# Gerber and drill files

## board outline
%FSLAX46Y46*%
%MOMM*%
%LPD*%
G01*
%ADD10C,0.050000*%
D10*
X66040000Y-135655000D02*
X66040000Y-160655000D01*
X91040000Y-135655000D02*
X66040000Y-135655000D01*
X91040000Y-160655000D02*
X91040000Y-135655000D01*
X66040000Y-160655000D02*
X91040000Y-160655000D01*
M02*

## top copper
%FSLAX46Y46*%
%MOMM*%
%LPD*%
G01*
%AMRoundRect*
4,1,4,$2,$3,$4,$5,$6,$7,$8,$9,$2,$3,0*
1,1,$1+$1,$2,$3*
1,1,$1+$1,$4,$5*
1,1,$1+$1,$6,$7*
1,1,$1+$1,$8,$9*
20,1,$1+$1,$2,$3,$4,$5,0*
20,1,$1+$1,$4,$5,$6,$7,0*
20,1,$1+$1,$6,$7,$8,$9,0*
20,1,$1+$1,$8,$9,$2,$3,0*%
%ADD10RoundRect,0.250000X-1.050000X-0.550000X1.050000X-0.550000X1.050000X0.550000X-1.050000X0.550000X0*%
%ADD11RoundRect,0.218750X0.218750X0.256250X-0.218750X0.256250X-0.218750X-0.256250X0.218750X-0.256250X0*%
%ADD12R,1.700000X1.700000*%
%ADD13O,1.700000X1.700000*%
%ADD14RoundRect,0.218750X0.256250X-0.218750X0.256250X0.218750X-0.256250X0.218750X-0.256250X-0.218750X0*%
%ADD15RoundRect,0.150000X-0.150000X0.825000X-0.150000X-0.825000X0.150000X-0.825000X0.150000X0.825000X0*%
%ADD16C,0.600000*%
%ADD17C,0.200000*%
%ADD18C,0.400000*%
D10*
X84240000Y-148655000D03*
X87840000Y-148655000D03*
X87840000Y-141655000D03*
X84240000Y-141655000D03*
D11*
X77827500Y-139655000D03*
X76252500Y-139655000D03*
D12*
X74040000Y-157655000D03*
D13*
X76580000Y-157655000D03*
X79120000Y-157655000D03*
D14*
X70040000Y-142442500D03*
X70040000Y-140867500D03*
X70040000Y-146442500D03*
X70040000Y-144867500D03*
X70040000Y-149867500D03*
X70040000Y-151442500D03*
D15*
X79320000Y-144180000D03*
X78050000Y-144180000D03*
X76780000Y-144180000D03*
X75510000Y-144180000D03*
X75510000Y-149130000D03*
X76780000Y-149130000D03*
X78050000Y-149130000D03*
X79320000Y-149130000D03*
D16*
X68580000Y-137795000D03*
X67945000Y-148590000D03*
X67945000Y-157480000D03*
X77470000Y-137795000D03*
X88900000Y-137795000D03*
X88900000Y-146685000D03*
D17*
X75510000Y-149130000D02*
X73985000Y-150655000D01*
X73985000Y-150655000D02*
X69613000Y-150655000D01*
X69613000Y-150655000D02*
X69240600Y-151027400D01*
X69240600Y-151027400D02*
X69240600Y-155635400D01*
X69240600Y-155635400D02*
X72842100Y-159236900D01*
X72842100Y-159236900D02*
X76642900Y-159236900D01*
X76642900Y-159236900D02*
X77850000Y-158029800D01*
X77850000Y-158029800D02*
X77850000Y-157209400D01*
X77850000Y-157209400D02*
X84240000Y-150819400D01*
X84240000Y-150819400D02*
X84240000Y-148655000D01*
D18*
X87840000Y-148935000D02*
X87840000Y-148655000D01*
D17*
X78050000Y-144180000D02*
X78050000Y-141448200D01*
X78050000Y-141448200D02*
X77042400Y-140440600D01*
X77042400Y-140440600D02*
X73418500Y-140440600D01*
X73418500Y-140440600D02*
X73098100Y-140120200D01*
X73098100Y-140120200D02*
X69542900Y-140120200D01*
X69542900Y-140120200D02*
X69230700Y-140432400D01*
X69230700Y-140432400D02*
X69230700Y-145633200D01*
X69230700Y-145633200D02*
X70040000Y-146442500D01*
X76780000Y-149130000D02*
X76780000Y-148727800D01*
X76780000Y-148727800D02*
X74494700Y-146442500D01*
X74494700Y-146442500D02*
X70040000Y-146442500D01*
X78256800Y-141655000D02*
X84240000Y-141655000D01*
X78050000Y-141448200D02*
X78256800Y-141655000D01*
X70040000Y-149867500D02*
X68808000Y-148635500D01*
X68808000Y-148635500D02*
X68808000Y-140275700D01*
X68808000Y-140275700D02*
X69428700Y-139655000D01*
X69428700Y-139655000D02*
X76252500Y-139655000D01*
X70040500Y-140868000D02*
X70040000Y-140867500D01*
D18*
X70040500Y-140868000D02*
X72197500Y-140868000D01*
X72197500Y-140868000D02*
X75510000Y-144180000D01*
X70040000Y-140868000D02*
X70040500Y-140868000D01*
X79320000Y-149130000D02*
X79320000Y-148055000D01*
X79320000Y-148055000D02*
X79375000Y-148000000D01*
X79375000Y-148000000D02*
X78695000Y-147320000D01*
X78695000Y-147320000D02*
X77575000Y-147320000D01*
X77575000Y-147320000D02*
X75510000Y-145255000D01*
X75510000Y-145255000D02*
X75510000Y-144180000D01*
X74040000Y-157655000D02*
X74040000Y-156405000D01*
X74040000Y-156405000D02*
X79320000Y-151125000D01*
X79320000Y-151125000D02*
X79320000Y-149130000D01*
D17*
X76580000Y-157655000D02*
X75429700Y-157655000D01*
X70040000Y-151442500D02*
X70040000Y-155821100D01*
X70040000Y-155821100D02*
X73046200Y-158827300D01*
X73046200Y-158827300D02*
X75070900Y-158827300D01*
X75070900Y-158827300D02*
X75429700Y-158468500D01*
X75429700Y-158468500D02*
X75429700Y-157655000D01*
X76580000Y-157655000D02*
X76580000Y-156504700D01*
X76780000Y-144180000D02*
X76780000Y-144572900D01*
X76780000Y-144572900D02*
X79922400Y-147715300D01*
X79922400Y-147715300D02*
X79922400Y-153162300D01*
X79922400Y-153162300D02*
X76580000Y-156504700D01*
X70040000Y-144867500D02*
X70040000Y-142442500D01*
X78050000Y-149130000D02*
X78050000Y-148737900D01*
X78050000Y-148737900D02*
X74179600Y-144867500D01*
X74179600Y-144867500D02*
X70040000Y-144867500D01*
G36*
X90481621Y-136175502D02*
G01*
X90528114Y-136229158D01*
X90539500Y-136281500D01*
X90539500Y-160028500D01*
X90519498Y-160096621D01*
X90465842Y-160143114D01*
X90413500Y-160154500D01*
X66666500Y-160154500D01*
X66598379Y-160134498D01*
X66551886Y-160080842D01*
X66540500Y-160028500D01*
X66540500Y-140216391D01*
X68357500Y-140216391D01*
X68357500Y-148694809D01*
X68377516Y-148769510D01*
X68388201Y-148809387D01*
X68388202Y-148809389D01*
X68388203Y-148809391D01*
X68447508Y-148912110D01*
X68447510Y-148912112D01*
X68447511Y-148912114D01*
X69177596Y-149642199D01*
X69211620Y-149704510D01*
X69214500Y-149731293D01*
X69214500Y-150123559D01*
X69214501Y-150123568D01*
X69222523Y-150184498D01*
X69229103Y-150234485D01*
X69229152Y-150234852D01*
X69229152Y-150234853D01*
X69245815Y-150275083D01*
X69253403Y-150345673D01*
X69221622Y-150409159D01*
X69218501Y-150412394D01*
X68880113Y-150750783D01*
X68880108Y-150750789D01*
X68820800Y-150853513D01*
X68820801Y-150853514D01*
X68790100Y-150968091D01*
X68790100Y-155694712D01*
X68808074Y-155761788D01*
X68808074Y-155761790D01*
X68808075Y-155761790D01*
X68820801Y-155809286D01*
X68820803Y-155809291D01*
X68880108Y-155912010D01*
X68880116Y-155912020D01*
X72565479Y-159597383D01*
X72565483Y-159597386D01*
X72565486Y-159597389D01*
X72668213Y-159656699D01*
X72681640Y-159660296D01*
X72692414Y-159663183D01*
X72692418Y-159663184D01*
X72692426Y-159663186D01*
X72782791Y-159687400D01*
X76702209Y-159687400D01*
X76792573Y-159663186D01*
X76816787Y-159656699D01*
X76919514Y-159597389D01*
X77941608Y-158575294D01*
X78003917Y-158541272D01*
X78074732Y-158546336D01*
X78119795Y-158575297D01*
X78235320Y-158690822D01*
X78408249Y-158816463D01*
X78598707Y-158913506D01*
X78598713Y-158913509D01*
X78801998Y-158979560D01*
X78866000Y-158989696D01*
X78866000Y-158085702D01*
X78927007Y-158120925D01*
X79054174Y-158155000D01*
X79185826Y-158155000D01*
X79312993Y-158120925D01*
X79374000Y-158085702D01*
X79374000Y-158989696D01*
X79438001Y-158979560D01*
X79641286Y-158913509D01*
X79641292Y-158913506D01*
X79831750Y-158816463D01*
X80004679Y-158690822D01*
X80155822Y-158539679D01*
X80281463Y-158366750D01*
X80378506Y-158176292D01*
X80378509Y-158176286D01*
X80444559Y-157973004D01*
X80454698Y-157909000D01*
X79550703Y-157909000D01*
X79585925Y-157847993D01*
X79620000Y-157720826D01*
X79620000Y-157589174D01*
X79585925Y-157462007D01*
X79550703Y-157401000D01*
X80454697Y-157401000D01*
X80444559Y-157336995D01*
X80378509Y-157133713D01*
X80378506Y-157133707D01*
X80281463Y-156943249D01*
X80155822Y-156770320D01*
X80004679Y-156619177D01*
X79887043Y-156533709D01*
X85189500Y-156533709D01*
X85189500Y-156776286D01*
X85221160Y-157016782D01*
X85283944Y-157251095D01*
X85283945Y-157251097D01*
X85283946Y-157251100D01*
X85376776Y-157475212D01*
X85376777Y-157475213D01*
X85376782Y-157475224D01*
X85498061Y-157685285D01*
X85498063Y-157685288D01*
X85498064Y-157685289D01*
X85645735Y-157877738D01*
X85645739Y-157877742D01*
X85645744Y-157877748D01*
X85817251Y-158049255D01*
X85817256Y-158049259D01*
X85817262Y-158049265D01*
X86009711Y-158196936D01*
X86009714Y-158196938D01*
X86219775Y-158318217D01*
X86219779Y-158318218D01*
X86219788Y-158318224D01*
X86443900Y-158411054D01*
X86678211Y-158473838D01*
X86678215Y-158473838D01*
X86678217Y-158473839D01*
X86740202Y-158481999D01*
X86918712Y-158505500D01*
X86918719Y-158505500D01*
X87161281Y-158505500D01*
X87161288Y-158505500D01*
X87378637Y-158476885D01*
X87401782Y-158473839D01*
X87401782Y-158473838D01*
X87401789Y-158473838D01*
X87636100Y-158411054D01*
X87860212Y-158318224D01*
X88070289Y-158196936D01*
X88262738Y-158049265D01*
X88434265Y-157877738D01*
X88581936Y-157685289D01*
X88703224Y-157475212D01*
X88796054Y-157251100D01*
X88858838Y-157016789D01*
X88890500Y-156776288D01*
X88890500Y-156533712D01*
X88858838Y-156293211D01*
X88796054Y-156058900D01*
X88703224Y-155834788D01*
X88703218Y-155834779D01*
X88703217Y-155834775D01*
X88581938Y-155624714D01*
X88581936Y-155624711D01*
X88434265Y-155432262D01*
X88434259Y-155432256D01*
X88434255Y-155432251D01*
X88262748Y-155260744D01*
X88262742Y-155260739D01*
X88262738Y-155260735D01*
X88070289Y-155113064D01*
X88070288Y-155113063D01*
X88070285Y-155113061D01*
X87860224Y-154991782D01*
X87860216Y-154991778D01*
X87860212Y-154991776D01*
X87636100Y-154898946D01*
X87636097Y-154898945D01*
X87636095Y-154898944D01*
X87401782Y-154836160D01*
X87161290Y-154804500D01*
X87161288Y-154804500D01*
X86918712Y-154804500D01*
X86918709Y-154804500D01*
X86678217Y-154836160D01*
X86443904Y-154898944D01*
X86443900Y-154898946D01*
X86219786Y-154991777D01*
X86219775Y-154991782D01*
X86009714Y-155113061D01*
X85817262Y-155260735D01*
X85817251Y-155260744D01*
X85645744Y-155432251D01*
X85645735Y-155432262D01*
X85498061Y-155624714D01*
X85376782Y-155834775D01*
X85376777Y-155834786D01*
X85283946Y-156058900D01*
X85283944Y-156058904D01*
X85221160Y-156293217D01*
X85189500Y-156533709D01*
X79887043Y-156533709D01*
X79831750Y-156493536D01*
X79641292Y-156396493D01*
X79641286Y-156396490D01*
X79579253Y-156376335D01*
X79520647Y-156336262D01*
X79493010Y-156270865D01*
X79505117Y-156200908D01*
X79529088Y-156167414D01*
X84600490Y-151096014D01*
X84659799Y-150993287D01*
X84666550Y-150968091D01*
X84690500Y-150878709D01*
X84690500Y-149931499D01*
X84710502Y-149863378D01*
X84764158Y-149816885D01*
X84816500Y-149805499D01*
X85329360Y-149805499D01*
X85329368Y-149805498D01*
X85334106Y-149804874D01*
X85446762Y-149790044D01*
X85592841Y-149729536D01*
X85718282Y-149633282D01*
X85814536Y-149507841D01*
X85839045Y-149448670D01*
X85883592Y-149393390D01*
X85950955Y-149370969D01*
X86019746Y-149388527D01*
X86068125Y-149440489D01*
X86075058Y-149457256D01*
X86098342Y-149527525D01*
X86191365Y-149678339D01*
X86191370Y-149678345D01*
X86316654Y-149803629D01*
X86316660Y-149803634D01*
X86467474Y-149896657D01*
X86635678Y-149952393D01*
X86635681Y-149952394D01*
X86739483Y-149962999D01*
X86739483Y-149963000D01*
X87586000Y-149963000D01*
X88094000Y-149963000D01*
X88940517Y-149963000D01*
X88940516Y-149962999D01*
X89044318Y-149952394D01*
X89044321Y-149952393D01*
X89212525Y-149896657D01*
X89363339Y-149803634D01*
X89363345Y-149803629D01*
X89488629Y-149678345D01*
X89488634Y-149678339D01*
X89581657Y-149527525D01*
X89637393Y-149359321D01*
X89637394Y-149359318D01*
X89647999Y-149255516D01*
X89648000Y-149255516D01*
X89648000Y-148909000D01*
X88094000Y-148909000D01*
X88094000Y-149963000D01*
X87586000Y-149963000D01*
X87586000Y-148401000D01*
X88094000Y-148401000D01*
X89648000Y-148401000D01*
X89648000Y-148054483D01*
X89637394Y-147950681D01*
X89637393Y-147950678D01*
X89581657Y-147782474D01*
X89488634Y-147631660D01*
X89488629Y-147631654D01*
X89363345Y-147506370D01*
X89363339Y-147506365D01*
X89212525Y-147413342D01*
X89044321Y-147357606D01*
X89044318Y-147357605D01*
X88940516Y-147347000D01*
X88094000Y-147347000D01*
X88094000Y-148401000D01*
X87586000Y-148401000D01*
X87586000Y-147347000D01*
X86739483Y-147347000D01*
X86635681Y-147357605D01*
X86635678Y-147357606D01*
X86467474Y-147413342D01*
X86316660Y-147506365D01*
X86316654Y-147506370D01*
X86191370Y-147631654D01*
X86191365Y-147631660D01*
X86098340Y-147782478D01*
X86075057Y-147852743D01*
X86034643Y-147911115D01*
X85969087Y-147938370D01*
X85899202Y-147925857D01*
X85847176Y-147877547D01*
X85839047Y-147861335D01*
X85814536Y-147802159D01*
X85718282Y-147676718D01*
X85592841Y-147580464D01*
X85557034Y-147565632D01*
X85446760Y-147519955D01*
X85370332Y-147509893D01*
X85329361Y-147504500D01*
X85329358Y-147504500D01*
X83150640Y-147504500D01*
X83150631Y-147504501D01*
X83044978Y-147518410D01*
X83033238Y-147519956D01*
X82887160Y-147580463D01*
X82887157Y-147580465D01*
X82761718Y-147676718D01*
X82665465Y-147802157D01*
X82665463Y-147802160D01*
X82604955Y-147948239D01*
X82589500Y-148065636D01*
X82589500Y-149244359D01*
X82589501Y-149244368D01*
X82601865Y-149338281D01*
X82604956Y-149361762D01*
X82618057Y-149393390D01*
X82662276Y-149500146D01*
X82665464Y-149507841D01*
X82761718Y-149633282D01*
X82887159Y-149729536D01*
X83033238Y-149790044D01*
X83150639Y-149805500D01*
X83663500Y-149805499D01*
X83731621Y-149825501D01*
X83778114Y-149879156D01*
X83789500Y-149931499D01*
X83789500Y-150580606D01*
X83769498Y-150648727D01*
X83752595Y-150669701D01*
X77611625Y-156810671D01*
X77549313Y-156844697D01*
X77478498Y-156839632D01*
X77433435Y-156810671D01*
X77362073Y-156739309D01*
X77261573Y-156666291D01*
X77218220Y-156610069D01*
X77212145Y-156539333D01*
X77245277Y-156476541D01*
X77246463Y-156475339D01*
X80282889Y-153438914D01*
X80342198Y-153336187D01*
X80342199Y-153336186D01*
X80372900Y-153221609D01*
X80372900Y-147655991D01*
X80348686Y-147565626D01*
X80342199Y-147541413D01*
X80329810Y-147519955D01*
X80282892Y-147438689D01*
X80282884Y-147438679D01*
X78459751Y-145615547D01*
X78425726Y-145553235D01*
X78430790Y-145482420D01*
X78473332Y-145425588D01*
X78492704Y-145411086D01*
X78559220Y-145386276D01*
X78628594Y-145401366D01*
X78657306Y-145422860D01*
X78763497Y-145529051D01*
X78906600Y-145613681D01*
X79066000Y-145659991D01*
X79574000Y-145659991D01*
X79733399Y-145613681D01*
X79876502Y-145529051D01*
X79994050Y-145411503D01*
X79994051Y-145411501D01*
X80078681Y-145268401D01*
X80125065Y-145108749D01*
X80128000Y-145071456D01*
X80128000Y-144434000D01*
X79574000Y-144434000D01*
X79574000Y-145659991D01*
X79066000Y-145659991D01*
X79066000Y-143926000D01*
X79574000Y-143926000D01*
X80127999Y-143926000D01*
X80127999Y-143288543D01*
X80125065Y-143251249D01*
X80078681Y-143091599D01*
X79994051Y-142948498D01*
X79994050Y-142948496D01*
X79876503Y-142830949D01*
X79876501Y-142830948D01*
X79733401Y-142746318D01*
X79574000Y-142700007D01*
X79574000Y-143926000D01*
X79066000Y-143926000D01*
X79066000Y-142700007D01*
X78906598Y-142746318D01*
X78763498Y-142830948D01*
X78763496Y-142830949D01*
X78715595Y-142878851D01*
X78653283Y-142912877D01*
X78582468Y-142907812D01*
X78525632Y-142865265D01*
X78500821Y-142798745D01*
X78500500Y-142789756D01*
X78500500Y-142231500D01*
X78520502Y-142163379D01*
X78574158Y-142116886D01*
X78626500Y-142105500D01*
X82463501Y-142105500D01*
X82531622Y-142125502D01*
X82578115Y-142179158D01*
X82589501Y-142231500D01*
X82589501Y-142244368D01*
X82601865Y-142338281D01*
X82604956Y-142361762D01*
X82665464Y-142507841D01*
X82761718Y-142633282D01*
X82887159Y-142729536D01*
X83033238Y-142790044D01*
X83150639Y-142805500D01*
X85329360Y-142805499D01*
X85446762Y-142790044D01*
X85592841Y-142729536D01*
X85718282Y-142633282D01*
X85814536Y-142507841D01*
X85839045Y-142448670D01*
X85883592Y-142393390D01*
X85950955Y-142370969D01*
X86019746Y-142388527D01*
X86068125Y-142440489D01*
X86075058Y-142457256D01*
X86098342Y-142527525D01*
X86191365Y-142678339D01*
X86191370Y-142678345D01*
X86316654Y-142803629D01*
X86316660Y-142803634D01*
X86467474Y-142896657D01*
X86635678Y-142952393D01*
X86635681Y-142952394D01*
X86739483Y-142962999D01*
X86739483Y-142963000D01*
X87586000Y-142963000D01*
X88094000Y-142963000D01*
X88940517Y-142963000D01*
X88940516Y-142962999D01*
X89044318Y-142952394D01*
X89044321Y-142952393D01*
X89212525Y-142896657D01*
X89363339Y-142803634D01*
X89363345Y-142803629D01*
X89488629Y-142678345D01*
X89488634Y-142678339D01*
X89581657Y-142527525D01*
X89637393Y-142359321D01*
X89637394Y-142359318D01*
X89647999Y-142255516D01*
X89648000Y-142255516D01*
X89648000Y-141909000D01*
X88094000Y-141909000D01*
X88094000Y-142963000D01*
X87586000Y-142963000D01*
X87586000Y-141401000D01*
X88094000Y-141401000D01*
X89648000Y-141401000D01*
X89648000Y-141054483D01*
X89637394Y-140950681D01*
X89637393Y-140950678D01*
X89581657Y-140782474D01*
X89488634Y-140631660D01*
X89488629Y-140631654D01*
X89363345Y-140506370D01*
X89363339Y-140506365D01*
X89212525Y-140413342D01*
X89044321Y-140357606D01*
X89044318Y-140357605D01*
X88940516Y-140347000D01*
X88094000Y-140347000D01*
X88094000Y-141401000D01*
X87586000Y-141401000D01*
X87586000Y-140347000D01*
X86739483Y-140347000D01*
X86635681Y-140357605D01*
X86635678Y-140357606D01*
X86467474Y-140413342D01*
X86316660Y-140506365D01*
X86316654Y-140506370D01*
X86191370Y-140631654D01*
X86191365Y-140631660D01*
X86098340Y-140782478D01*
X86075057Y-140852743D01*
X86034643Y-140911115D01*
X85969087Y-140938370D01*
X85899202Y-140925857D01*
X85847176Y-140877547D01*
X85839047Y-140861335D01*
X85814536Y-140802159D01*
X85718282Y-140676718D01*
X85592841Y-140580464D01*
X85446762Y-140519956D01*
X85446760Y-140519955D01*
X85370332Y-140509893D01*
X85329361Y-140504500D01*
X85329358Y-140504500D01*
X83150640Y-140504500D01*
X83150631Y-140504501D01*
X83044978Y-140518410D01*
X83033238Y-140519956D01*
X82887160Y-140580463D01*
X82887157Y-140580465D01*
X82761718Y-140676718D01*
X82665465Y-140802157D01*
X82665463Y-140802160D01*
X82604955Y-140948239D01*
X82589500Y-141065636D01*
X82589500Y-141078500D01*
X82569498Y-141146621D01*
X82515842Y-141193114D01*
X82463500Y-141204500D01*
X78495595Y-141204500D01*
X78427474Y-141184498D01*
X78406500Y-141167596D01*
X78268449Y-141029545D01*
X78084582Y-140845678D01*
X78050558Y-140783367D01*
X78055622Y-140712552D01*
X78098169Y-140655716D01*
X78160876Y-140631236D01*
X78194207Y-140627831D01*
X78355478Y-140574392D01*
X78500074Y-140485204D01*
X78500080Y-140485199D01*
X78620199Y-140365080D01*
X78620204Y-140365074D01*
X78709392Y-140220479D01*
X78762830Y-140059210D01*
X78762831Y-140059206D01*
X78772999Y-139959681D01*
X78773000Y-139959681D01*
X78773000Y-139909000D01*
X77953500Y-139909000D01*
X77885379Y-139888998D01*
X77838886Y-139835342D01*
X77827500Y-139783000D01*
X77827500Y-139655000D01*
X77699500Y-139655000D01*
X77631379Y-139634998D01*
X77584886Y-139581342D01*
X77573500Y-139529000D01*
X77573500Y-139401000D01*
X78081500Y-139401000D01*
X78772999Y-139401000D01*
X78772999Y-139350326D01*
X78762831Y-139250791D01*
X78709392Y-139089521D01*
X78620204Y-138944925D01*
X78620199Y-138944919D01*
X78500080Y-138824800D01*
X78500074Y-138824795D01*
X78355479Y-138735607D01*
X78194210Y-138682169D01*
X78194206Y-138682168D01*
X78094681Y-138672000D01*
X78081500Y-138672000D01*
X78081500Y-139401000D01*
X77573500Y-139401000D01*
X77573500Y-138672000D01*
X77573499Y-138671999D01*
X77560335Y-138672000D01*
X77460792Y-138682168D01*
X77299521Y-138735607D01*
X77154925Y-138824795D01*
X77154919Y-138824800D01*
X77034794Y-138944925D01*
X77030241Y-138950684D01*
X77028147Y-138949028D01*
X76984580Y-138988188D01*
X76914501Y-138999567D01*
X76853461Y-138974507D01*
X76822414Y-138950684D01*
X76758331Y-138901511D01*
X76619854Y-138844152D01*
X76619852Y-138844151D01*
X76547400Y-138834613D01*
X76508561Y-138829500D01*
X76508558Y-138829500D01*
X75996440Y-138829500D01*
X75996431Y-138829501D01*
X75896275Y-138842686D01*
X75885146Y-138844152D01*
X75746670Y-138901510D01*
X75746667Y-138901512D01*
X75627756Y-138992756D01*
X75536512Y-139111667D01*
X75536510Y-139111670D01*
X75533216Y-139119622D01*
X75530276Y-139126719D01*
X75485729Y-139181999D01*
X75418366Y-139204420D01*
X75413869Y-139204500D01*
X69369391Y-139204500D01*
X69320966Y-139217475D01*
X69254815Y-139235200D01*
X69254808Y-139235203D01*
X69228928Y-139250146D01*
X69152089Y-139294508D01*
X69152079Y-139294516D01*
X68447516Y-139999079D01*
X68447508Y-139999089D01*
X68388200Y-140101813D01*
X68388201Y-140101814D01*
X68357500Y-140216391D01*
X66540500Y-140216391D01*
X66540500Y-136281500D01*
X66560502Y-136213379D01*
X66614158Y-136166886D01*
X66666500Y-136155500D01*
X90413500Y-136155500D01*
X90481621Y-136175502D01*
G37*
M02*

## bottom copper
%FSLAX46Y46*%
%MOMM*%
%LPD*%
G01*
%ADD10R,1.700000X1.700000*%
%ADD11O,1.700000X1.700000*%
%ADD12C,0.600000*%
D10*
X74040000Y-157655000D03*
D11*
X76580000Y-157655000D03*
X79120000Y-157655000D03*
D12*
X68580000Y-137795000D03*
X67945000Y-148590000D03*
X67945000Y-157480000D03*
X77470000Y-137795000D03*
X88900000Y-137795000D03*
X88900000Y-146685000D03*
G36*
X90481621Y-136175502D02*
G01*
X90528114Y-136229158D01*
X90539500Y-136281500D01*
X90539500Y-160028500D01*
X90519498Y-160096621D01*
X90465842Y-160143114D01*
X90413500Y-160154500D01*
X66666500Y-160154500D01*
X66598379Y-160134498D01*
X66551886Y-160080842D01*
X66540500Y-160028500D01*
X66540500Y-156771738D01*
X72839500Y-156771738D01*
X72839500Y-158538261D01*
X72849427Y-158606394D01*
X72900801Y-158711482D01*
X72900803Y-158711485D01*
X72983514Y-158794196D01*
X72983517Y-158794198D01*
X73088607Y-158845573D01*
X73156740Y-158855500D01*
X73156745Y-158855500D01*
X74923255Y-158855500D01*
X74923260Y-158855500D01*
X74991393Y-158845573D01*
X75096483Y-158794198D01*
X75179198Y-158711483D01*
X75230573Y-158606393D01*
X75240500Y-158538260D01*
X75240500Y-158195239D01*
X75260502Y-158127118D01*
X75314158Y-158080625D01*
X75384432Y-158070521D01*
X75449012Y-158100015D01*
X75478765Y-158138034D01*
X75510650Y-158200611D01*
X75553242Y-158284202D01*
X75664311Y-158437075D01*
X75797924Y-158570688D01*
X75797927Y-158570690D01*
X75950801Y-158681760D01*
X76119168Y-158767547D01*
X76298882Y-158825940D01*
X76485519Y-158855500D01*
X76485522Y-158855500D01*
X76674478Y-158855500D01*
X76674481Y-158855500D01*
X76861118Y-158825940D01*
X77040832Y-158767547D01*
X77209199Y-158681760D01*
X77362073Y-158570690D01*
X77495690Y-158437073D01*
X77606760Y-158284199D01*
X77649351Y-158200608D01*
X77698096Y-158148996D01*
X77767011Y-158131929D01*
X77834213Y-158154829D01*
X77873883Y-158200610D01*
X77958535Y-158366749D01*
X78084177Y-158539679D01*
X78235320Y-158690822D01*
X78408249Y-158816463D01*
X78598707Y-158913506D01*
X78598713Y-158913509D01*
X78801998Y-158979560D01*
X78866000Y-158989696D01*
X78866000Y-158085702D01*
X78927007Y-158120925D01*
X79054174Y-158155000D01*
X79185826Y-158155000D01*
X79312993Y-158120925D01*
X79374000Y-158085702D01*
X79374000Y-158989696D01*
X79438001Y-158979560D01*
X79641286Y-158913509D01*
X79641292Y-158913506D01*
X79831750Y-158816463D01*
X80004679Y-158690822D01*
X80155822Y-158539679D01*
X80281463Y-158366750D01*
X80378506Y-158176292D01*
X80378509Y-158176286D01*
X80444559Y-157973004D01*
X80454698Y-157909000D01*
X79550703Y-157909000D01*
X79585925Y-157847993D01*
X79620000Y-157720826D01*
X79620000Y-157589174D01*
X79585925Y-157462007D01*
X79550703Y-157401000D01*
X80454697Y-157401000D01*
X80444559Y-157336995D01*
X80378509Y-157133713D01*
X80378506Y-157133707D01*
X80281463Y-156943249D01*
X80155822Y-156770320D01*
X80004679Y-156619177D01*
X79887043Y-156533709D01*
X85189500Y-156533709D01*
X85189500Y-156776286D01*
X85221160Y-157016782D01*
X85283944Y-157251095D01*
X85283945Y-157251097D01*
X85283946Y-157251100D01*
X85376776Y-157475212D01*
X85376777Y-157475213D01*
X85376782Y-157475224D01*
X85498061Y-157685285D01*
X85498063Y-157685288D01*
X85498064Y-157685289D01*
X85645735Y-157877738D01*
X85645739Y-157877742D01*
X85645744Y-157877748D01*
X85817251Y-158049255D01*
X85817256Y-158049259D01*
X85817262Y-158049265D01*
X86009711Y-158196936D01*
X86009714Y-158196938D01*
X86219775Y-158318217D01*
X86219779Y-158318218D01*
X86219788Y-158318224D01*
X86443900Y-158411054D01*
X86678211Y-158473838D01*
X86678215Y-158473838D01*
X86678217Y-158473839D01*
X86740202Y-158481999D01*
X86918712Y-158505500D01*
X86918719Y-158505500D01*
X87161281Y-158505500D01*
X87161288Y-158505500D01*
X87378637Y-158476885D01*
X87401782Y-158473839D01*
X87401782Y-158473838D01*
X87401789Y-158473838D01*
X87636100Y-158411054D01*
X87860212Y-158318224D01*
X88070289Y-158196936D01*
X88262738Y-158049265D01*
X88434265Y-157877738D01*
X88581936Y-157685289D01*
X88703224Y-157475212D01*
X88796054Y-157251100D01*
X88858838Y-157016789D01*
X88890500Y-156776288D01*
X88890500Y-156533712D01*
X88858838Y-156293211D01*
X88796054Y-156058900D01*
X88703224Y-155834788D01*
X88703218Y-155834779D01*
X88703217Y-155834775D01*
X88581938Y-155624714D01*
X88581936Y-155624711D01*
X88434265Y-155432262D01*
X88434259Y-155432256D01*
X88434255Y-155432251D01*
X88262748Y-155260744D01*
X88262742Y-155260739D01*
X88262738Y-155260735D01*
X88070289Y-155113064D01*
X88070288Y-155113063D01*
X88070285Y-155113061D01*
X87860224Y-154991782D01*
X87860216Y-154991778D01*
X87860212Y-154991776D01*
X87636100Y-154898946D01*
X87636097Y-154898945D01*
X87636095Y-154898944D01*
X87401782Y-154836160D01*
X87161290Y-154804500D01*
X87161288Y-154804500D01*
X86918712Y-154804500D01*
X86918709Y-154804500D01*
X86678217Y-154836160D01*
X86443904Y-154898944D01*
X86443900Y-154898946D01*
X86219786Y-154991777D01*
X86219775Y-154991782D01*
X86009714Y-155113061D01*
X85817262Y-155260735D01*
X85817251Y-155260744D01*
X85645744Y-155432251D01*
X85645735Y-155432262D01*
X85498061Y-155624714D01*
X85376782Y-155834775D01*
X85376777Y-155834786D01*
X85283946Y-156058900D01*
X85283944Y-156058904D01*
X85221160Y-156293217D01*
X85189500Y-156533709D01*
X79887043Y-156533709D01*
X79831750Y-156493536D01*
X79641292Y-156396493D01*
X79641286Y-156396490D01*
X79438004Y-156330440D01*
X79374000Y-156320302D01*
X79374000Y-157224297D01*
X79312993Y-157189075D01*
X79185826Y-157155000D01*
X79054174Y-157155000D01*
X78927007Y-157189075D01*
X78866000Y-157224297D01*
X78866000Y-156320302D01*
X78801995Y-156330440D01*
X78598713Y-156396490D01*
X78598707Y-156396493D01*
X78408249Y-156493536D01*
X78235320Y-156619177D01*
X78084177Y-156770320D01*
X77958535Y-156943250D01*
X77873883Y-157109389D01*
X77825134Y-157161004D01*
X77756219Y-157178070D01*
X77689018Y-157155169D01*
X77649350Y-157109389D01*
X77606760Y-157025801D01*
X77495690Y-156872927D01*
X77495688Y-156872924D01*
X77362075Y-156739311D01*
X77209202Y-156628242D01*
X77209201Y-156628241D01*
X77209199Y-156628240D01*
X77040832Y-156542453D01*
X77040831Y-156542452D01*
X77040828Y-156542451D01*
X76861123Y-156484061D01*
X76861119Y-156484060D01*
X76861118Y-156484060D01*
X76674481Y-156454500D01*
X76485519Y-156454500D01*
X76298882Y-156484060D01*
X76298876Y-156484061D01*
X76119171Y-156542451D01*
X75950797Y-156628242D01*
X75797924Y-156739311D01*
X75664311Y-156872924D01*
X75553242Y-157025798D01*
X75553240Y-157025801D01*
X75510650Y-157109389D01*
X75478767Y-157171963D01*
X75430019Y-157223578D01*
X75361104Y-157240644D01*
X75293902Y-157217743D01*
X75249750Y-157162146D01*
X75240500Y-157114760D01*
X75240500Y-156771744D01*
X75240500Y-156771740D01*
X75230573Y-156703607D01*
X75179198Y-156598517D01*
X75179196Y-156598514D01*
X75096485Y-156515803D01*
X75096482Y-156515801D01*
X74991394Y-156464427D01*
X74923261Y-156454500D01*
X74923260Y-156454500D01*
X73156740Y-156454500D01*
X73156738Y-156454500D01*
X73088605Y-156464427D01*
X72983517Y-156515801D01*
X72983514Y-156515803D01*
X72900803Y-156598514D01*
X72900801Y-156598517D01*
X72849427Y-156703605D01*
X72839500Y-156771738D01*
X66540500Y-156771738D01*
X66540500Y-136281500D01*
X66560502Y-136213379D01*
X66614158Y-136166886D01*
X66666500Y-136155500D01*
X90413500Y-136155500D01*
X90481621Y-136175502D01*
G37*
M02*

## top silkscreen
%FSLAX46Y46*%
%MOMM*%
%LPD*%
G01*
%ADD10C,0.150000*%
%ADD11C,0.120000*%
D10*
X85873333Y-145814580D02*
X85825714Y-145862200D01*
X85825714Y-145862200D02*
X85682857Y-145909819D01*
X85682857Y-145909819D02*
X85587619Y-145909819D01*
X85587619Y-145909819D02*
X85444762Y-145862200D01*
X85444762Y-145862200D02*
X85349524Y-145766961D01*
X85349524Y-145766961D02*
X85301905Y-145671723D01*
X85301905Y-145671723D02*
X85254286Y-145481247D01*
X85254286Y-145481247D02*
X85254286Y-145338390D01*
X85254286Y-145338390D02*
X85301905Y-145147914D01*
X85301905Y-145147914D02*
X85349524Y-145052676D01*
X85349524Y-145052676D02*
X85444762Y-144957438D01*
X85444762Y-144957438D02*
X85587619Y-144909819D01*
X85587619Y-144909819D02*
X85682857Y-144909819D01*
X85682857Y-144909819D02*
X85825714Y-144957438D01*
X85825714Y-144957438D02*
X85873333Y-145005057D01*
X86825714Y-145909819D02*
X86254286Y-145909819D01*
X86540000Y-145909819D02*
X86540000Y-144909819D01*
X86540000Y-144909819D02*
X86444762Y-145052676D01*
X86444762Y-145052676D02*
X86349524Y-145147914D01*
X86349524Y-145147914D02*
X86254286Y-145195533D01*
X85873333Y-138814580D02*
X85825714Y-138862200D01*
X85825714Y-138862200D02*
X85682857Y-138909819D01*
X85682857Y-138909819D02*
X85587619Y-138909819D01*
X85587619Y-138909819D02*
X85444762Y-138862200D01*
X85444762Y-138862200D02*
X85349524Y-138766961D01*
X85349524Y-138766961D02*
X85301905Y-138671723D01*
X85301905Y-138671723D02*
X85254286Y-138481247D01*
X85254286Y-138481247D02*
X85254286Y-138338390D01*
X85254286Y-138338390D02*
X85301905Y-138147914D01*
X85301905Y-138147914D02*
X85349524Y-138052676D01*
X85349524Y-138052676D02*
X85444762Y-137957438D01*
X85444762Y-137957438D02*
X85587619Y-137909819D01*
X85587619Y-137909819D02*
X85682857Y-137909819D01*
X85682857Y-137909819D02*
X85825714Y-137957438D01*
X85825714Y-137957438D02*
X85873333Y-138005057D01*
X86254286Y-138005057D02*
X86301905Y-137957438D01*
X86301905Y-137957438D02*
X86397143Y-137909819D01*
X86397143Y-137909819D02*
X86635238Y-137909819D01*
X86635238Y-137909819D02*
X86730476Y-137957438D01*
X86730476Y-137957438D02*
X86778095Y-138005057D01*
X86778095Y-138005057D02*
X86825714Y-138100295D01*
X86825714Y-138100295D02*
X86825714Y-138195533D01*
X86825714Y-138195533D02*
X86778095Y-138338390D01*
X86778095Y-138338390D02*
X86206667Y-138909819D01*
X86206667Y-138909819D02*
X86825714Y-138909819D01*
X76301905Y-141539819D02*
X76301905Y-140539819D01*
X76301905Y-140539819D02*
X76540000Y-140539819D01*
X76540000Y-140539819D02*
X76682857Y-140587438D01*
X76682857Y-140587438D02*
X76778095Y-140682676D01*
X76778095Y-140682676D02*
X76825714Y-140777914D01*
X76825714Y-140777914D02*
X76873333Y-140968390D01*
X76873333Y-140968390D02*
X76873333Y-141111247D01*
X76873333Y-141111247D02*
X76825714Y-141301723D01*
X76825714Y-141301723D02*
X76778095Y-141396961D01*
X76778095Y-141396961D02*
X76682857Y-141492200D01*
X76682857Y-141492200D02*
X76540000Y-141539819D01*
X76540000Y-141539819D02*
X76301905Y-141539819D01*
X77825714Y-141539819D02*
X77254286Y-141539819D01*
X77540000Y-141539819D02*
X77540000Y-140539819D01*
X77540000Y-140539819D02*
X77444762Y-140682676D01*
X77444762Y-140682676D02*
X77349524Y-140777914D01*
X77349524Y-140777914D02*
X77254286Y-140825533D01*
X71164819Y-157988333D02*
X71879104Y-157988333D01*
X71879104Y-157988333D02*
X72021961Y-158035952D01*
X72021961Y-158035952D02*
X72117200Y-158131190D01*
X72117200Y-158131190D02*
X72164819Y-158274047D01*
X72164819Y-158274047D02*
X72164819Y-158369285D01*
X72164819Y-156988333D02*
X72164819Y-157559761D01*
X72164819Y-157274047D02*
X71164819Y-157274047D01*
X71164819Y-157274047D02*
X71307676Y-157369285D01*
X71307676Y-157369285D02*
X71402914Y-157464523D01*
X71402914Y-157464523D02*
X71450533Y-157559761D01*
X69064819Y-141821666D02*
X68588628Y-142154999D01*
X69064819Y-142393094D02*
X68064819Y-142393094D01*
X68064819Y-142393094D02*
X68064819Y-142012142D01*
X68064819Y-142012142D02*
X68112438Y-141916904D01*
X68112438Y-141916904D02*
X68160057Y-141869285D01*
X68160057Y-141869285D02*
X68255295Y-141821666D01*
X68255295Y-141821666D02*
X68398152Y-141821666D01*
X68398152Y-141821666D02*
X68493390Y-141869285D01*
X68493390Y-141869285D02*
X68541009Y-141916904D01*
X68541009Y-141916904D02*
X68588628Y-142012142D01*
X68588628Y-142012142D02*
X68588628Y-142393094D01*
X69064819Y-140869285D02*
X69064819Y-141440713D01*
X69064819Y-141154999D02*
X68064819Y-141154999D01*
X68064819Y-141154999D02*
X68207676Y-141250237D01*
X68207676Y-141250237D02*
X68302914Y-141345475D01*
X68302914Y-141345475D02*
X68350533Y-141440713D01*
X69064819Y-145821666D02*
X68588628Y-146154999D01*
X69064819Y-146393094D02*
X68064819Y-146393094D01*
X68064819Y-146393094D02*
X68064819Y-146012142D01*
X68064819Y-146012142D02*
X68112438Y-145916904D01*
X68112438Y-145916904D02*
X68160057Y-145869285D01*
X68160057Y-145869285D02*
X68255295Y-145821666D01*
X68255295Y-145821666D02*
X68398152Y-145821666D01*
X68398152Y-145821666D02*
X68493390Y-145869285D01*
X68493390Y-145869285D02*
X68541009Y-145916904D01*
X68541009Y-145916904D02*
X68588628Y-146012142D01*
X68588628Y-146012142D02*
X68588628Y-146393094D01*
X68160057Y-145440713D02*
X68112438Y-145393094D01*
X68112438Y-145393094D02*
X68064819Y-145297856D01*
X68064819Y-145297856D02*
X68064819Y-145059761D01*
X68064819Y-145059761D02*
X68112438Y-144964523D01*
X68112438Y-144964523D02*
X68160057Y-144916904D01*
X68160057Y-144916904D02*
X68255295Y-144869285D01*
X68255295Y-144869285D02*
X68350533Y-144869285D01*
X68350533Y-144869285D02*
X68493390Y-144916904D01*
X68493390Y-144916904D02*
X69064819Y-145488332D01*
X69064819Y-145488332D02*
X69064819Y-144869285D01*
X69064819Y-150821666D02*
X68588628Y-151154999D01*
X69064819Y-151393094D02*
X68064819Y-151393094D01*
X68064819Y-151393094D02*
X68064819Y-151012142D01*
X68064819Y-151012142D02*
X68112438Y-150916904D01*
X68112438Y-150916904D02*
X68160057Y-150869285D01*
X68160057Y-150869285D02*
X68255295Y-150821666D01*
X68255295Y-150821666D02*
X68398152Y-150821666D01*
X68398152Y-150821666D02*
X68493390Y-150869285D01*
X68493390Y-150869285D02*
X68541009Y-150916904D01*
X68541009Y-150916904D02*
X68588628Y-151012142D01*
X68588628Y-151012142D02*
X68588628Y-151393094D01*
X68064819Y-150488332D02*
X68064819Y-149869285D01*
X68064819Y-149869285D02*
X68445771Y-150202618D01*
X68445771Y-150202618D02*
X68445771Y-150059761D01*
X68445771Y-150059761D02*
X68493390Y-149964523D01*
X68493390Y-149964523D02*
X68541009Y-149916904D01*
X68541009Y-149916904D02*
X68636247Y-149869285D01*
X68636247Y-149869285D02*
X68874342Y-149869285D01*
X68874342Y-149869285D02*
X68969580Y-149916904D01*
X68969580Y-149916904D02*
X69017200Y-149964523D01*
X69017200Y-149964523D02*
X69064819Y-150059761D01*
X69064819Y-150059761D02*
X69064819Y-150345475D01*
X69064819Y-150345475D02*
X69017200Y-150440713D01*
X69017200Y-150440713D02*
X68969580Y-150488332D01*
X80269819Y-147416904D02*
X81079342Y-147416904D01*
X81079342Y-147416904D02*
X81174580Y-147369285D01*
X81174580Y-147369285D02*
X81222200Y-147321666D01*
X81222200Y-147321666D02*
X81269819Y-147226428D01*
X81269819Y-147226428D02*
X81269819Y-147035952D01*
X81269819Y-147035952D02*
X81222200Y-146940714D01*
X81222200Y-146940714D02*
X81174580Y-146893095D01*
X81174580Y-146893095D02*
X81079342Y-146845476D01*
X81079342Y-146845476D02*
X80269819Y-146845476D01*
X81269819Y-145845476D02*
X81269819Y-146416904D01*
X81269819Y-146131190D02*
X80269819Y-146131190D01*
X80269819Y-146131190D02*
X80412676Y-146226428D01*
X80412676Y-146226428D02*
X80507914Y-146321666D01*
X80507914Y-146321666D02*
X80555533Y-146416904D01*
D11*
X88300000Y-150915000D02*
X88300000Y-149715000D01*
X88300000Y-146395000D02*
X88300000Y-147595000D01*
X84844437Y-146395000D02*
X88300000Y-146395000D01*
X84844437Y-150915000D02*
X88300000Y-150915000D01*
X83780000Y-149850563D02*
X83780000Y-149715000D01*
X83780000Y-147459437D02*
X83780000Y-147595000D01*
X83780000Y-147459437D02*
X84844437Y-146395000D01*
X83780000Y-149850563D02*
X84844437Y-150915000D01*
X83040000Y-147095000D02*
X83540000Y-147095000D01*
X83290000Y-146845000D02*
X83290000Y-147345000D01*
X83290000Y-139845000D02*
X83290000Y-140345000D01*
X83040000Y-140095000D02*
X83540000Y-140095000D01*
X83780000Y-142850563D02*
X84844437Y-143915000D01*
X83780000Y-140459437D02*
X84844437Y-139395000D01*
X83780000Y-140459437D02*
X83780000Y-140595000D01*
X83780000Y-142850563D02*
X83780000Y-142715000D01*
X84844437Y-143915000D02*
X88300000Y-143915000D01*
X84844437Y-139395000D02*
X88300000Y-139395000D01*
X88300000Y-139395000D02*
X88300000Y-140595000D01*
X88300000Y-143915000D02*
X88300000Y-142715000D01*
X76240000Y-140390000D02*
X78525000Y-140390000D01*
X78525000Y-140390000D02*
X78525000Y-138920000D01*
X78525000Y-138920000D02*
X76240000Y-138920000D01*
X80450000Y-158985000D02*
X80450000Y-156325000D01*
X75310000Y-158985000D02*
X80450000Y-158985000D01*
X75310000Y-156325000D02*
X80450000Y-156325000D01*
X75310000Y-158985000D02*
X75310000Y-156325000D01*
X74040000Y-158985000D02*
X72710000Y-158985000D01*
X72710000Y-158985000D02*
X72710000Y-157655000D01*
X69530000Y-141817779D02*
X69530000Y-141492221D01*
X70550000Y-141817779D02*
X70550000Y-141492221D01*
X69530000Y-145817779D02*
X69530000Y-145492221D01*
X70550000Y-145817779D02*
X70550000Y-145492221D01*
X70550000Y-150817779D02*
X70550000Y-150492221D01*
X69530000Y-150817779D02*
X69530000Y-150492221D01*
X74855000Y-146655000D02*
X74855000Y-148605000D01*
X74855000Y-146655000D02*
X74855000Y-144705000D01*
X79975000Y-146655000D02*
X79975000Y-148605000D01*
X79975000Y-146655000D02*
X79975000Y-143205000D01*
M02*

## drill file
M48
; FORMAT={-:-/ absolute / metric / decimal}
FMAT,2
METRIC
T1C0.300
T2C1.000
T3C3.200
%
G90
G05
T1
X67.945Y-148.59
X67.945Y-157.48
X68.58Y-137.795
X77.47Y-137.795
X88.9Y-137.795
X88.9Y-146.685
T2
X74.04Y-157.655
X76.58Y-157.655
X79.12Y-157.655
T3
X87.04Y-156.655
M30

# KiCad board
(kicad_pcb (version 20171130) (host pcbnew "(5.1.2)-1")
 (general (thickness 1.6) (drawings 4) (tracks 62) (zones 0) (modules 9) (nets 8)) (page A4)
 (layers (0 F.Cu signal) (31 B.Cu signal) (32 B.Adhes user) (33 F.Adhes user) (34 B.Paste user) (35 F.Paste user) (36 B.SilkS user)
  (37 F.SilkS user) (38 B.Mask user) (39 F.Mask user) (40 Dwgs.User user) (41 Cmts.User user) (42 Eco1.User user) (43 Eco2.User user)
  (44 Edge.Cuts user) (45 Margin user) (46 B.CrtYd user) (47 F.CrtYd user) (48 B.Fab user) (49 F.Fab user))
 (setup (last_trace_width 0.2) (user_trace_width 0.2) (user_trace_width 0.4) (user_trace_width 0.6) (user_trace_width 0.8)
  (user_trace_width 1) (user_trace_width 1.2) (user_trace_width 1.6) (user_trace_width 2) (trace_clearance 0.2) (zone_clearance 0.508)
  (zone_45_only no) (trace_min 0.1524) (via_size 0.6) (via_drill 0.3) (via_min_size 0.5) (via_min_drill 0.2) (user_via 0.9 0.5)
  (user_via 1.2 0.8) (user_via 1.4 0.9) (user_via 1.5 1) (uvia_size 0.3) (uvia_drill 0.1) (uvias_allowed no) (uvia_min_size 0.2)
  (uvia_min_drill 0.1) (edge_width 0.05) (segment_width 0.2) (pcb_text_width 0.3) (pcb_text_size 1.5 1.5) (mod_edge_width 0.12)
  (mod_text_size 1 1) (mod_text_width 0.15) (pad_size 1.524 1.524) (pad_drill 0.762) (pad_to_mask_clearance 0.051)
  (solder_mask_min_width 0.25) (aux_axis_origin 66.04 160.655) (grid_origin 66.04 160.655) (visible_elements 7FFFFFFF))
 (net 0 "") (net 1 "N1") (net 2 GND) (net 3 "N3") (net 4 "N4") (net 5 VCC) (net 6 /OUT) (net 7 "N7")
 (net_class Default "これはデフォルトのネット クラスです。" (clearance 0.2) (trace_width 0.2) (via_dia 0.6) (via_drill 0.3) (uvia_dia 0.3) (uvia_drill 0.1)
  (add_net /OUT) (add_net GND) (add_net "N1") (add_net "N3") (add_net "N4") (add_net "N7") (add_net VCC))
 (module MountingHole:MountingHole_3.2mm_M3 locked (layer F.Cu) (at 87.04 156.655)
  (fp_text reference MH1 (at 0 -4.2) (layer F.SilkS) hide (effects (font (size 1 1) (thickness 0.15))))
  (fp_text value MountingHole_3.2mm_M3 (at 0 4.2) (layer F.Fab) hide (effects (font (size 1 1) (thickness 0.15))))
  (pad 1 np_thru_hole circle (at 0 0) (size 3.2 3.2) (drill 3.2) (layers *.Cu *.Mask)))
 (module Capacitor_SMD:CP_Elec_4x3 (layer F.Cu) (at 86.04 148.655)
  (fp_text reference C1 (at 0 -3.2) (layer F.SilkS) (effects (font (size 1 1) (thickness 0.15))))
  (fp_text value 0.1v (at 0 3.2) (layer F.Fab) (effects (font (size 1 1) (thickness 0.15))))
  (fp_line (start 2.26 2.26) (end 2.26 1.06) (layer F.SilkS) (width 0.12))
  (fp_line (start 2.26 -2.26) (end 2.26 -1.06) (layer F.SilkS) (width 0.12))
  (fp_line (start -1.195563 -2.26) (end 2.26 -2.26) (layer F.SilkS) (width 0.12))
  (fp_line (start -1.195563 2.26) (end 2.26 2.26) (layer F.SilkS) (width 0.12))
  (fp_line (start -2.26 1.195563) (end -2.26 1.06) (layer F.SilkS) (width 0.12))
  (fp_line (start -2.26 -1.195563) (end -2.26 -1.06) (layer F.SilkS) (width 0.12))
  (fp_line (start -2.26 -1.195563) (end -1.195563 -2.26) (layer F.SilkS) (width 0.12))
  (fp_line (start -2.26 1.195563) (end -1.195563 2.26) (layer F.SilkS) (width 0.12))
  (fp_line (start -3 -1.56) (end -2.5 -1.56) (layer F.SilkS) (width 0.12))
  (fp_line (start -2.75 -1.81) (end -2.75 -1.31) (layer F.SilkS) (width 0.12))
  (pad 1 smd roundrect (at -1.8 0) (size 2.6 1.6) (layers F.Cu F.Paste F.Mask) (roundrect_rratio 0.15625) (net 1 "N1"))
  (pad 2 smd roundrect (at 1.8 0) (size 2.6 1.6) (layers F.Cu F.Paste F.Mask) (roundrect_rratio 0.15625) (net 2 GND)))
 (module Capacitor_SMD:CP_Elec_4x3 (layer F.Cu) (at 86.04 141.655)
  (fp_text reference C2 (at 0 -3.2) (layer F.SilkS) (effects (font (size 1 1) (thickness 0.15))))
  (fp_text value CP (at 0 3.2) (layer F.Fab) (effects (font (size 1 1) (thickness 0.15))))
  (fp_line (start -2.75 -1.81) (end -2.75 -1.31) (layer F.SilkS) (width 0.12))
  (fp_line (start -3 -1.56) (end -2.5 -1.56) (layer F.SilkS) (width 0.12))
  (fp_line (start -2.26 1.195563) (end -1.195563 2.26) (layer F.SilkS) (width 0.12))
  (fp_line (start -2.26 -1.195563) (end -1.195563 -2.26) (layer F.SilkS) (width 0.12))
  (fp_line (start -2.26 -1.195563) (end -2.26 -1.06) (layer F.SilkS) (width 0.12))
  (fp_line (start -2.26 1.195563) (end -2.26 1.06) (layer F.SilkS) (width 0.12))
  (fp_line (start -1.195563 2.26) (end 2.26 2.26) (layer F.SilkS) (width 0.12))
  (fp_line (start -1.195563 -2.26) (end 2.26 -2.26) (layer F.SilkS) (width 0.12))
  (fp_line (start 2.26 -2.26) (end 2.26 -1.06) (layer F.SilkS) (width 0.12))
  (fp_line (start 2.26 2.26) (end 2.26 1.06) (layer F.SilkS) (width 0.12))
  (pad 2 smd roundrect (at 1.8 0) (size 2.6 1.6) (layers F.Cu F.Paste F.Mask) (roundrect_rratio 0.15625) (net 2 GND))
  (pad 1 smd roundrect (at -1.8 0) (size 2.6 1.6) (layers F.Cu F.Paste F.Mask) (roundrect_rratio 0.15625) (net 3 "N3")))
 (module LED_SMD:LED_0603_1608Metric (layer F.Cu) (at 77.04 139.655 180)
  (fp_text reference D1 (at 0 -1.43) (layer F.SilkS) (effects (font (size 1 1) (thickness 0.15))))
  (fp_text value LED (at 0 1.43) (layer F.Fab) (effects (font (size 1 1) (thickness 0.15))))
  (fp_line (start 0.8 -0.735) (end -1.485 -0.735) (layer F.SilkS) (width 0.12))
  (fp_line (start -1.485 -0.735) (end -1.485 0.735) (layer F.SilkS) (width 0.12))
  (fp_line (start -1.485 0.735) (end 0.8 0.735) (layer F.SilkS) (width 0.12))
  (pad 1 smd roundrect (at -0.7875 0 180) (size 0.875 0.95) (layers F.Cu F.Paste F.Mask) (roundrect_rratio 0.25) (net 2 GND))
  (pad 2 smd roundrect (at 0.7875 0 180) (size 0.875 0.95) (layers F.Cu F.Paste F.Mask) (roundrect_rratio 0.25) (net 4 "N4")))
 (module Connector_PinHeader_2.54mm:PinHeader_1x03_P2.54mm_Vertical (layer F.Cu) (at 74.04 157.655 90)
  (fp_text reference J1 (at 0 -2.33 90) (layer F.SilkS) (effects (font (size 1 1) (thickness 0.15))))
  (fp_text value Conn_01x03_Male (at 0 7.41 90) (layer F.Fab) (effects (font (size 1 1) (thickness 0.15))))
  (fp_line (start -1.33 6.41) (end 1.33 6.41) (layer F.SilkS) (width 0.12))
  (fp_line (start -1.33 1.27) (end -1.33 6.41) (layer F.SilkS) (width 0.12))
  (fp_line (start 1.33 1.27) (end 1.33 6.41) (layer F.SilkS) (width 0.12))
  (fp_line (start -1.33 1.27) (end 1.33 1.27) (layer F.SilkS) (width 0.12))
  (fp_line (start -1.33 0) (end -1.33 -1.33) (layer F.SilkS) (width 0.12))
  (fp_line (start -1.33 -1.33) (end 0 -1.33) (layer F.SilkS) (width 0.12))
  (pad 1 thru_hole rect (at 0 0 90) (size 1.7 1.7) (drill 1) (layers *.Cu *.Mask) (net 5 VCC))
  (pad 2 thru_hole oval (at 0 2.54 90) (size 1.7 1.7) (drill 1) (layers *.Cu *.Mask) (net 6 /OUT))
  (pad 3 thru_hole oval (at 0 5.08 90) (size 1.7 1.7) (drill 1) (layers *.Cu *.Mask) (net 2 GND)))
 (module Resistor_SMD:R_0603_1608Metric (layer F.Cu) (at 70.04 141.655 90)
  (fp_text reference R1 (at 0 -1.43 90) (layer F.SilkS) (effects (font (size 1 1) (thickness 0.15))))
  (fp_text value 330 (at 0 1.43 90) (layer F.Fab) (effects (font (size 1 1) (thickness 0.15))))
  (fp_line (start -0.162779 -0.51) (end 0.162779 -0.51) (layer F.SilkS) (width 0.12))
  (fp_line (start -0.162779 0.51) (end 0.162779 0.51) (layer F.SilkS) (width 0.12))
  (pad 1 smd roundrect (at -0.7875 0 90) (size 0.875 0.95) (layers F.Cu F.Paste F.Mask) (roundrect_rratio 0.25) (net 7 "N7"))
  (pad 2 smd roundrect (at 0.7875 0 90) (size 0.875 0.95) (layers F.Cu F.Paste F.Mask) (roundrect_rratio 0.25) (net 5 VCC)))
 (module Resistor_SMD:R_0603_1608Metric (layer F.Cu) (at 70.04 145.655 90)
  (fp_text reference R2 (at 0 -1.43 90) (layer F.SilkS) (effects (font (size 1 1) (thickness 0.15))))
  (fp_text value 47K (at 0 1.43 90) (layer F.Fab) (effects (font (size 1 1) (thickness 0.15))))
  (fp_line (start -0.162779 -0.51) (end 0.162779 -0.51) (layer F.SilkS) (width 0.12))
  (fp_line (start -0.162779 0.51) (end 0.162779 0.51) (layer F.SilkS) (width 0.12))
  (pad 1 smd roundrect (at -0.7875 0 90) (size 0.875 0.95) (layers F.Cu F.Paste F.Mask) (roundrect_rratio 0.25) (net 3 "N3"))
  (pad 2 smd roundrect (at 0.7875 0 90) (size 0.875 0.95) (layers F.Cu F.Paste F.Mask) (roundrect_rratio 0.25) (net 7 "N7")))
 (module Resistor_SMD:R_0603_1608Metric (layer F.Cu) (at 70.04 150.655 90)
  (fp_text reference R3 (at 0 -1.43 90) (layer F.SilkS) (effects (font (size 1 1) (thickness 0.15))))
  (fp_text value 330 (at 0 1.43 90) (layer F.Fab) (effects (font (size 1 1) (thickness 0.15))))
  (fp_line (start -0.162779 0.51) (end 0.162779 0.51) (layer F.SilkS) (width 0.12))
  (fp_line (start -0.162779 -0.51) (end 0.162779 -0.51) (layer F.SilkS) (width 0.12))
  (pad 2 smd roundrect (at 0.7875 0 90) (size 0.875 0.95) (layers F.Cu F.Paste F.Mask) (roundrect_rratio 0.25) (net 4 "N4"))
  (pad 1 smd roundrect (at -0.7875 0 90) (size 0.875 0.95) (layers F.Cu F.Paste F.Mask) (roundrect_rratio 0.25) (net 6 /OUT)))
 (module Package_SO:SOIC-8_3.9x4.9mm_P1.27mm (layer F.Cu) (at 77.415 146.655 270)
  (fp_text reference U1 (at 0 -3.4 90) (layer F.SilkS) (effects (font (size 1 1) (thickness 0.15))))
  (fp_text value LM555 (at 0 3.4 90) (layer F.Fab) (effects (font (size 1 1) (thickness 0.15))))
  (fp_line (start 0 2.56) (end 1.95 2.56) (layer F.SilkS) (width 0.12))
  (fp_line (start 0 2.56) (end -1.95 2.56) (layer F.SilkS) (width 0.12))
  (fp_line (start 0 -2.56) (end 1.95 -2.56) (layer F.SilkS) (width 0.12))
  (fp_line (start 0 -2.56) (end -3.45 -2.56) (layer F.SilkS) (width 0.12))
  (pad 1 smd roundrect (at -2.475 -1.905 270) (size 1.95 0.6) (layers F.Cu F.Paste F.Mask) (roundrect_rratio 0.25) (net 2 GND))
  (pad 2 smd roundrect (at -2.475 -0.635 270) (size 1.95 0.6) (layers F.Cu F.Paste F.Mask) (roundrect_rratio 0.25) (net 3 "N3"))
  (pad 3 smd roundrect (at -2.475 0.635 270) (size 1.95 0.6) (layers F.Cu F.Paste F.Mask) (roundrect_rratio 0.25) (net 6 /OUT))
  (pad 4 smd roundrect (at -2.475 1.905 270) (size 1.95 0.6) (layers F.Cu F.Paste F.Mask) (roundrect_rratio 0.25) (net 5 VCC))
  (pad 5 smd roundrect (at 2.475 1.905 270) (size 1.95 0.6) (layers F.Cu F.Paste F.Mask) (roundrect_rratio 0.25) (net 1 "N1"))
  (pad 6 smd roundrect (at 2.475 0.635 270) (size 1.95 0.6) (layers F.Cu F.Paste F.Mask) (roundrect_rratio 0.25) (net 3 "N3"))
  (pad 7 smd roundrect (at 2.475 -0.635 270) (size 1.95 0.6) (layers F.Cu F.Paste F.Mask) (roundrect_rratio 0.25) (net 7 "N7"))
  (pad 8 smd roundrect (at 2.475 -1.905 270) (size 1.95 0.6) (layers F.Cu F.Paste F.Mask) (roundrect_rratio 0.25) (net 5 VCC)))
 (gr_line (start 66.04 135.655) (end 66.04 160.655) (layer Edge.Cuts) (width 0.05))
 (gr_line (start 91.04 135.655) (end 66.04 135.655) (layer Edge.Cuts) (width 0.05))
 (gr_line (start 91.04 160.655) (end 91.04 135.655) (layer Edge.Cuts) (width 0.05))
 (gr_line (start 66.04 160.655) (end 91.04 160.655) (layer Edge.Cuts) (width 0.05))
 (segment (start 75.51 149.13) (end 73.985 150.655) (width 0.2) (layer F.Cu) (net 1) (status 10))
 (segment (start 73.985 150.655) (end 69.613 150.655) (width 0.2) (layer F.Cu) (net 1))
 (segment (start 69.613 150.655) (end 69.2406 151.0274) (width 0.2) (layer F.Cu) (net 1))
 (segment (start 69.2406 151.0274) (end 69.2406 155.6354) (width 0.2) (layer F.Cu) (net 1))
 (segment (start 69.2406 155.6354) (end 72.8421 159.2369) (width 0.2) (layer F.Cu) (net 1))
 (segment (start 72.8421 159.2369) (end 76.6429 159.2369) (width 0.2) (layer F.Cu) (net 1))
 (segment (start 76.6429 159.2369) (end 77.85 158.0298) (width 0.2) (layer F.Cu) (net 1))
 (segment (start 77.85 158.0298) (end 77.85 157.2094) (width 0.2) (layer F.Cu) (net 1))
 (segment (start 77.85 157.2094) (end 84.24 150.8194) (width 0.2) (layer F.Cu) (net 1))
 (segment (start 84.24 150.8194) (end 84.24 148.655) (width 0.2) (layer F.Cu) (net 1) (status 20))
 (segment (start 87.84 148.935) (end 87.84 148.655) (width 0.4) (layer F.Cu) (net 2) (status 30))
 (via (at 68.58 137.795) (size 0.6) (drill 0.3) (layers F.Cu B.Cu) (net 2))
 (via (at 67.945 148.59) (size 0.6) (drill 0.3) (layers F.Cu B.Cu) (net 2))
 (via (at 67.945 157.48) (size 0.6) (drill 0.3) (layers F.Cu B.Cu) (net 2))
 (via (at 77.47 137.795) (size 0.6) (drill 0.3) (layers F.Cu B.Cu) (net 2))
 (via (at 88.9 137.795) (size 0.6) (drill 0.3) (layers F.Cu B.Cu) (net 2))
 (via (at 88.9 146.685) (size 0.6) (drill 0.3) (layers F.Cu B.Cu) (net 2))
 (segment (start 78.05 144.18) (end 78.05 141.4482) (width 0.2) (layer F.Cu) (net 3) (status 10))
 (segment (start 78.05 141.4482) (end 77.0424 140.4406) (width 0.2) (layer F.Cu) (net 3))
 (segment (start 77.0424 140.4406) (end 73.4185 140.4406) (width 0.2) (layer F.Cu) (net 3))
 (segment (start 73.4185 140.4406) (end 73.0981 140.1202) (width 0.2) (layer F.Cu) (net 3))
 (segment (start 73.0981 140.1202) (end 69.5429 140.1202) (width 0.2) (layer F.Cu) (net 3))
 (segment (start 69.5429 140.1202) (end 69.2307 140.4324) (width 0.2) (layer F.Cu) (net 3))
 (segment (start 69.2307 140.4324) (end 69.2307 145.6332) (width 0.2) (layer F.Cu) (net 3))
 (segment (start 69.2307 145.6332) (end 70.04 146.4425) (width 0.2) (layer F.Cu) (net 3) (status 20))
 (segment (start 76.78 149.13) (end 76.78 148.7278) (width 0.2) (layer F.Cu) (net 3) (status 30))
 (segment (start 76.78 148.7278) (end 74.4947 146.4425) (width 0.2) (layer F.Cu) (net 3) (status 10))
 (segment (start 74.4947 146.4425) (end 70.04 146.4425) (width 0.2) (layer F.Cu) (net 3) (status 20))
 (segment (start 78.2568 141.655) (end 84.24 141.655) (width 0.2) (layer F.Cu) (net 3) (status 20))
 (segment (start 78.05 141.4482) (end 78.2568 141.655) (width 0.2) (layer F.Cu) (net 3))
 (segment (start 70.04 149.8675) (end 68.808 148.6355) (width 0.2) (layer F.Cu) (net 4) (status 10))
 (segment (start 68.808 148.6355) (end 68.808 140.2757) (width 0.2) (layer F.Cu) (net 4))
 (segment (start 68.808 140.2757) (end 69.4287 139.655) (width 0.2) (layer F.Cu) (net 4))
 (segment (start 69.4287 139.655) (end 76.2525 139.655) (width 0.2) (layer F.Cu) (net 4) (status 20))
 (segment (start 70.0405 140.868) (end 70.04 140.8675) (width 0.2) (layer F.Cu) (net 5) (status 30))
 (segment (start 70.0405 140.868) (end 72.1975 140.868) (width 0.4) (layer F.Cu) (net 5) (status 10))
 (segment (start 72.1975 140.868) (end 75.51 144.18) (width 0.4) (layer F.Cu) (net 5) (status 20))
 (segment (start 70.04 140.868) (end 70.0405 140.868) (width 0.4) (layer F.Cu) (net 5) (status 30))
 (segment (start 79.32 149.13) (end 79.32 148.055) (width 0.4) (layer F.Cu) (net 5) (status 10))
 (segment (start 79.32 148.055) (end 79.375 148) (width 0.4) (layer F.Cu) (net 5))
 (segment (start 79.375 148) (end 78.695 147.32) (width 0.4) (layer F.Cu) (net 5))
 (segment (start 78.695 147.32) (end 77.575 147.32) (width 0.4) (layer F.Cu) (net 5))
 (segment (start 77.575 147.32) (end 75.51 145.255) (width 0.4) (layer F.Cu) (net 5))
 (segment (start 75.51 145.255) (end 75.51 144.18) (width 0.4) (layer F.Cu) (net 5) (status 20))
 (segment (start 74.04 157.655) (end 74.04 156.405) (width 0.4) (layer F.Cu) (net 5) (status 10))
 (segment (start 74.04 156.405) (end 79.32 151.125) (width 0.4) (layer F.Cu) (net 5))
 (segment (start 79.32 151.125) (end 79.32 149.13) (width 0.4) (layer F.Cu) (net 5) (status 20))
 (segment (start 76.58 157.655) (end 75.4297 157.655) (width 0.2) (layer F.Cu) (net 6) (status 10))
 (segment (start 70.04 151.4425) (end 70.04 155.8211) (width 0.2) (layer F.Cu) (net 6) (status 10))
 (segment (start 70.04 155.8211) (end 73.0462 158.8273) (width 0.2) (layer F.Cu) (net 6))
 (segment (start 73.0462 158.8273) (end 75.0709 158.8273) (width 0.2) (layer F.Cu) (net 6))
 (segment (start 75.0709 158.8273) (end 75.4297 158.4685) (width 0.2) (layer F.Cu) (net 6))
 (segment (start 75.4297 158.4685) (end 75.4297 157.655) (width 0.2) (layer F.Cu) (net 6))
 (segment (start 76.58 157.655) (end 76.58 156.5047) (width 0.2) (layer F.Cu) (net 6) (status 10))
 (segment (start 76.78 144.18) (end 76.78 144.5729) (width 0.2) (layer F.Cu) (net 6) (status 30))
 (segment (start 76.78 144.5729) (end 79.9224 147.7153) (width 0.2) (layer F.Cu) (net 6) (status 10))
 (segment (start 79.9224 147.7153) (end 79.9224 153.1623) (width 0.2) (layer F.Cu) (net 6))
 (segment (start 79.9224 153.1623) (end 76.58 156.5047) (width 0.2) (layer F.Cu) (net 6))
 (segment (start 70.04 144.8675) (end 70.04 142.4425) (width 0.2) (layer F.Cu) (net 7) (status 30))
 (segment (start 78.05 149.13) (end 78.05 148.7379) (width 0.2) (layer F.Cu) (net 7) (status 30))
 (segment (start 78.05 148.7379) (end 74.1796 144.8675) (width 0.2) (layer F.Cu) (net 7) (status 10))
 (segment (start 74.1796 144.8675) (end 70.04 144.8675) (width 0.2) (layer F.Cu) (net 7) (status 20))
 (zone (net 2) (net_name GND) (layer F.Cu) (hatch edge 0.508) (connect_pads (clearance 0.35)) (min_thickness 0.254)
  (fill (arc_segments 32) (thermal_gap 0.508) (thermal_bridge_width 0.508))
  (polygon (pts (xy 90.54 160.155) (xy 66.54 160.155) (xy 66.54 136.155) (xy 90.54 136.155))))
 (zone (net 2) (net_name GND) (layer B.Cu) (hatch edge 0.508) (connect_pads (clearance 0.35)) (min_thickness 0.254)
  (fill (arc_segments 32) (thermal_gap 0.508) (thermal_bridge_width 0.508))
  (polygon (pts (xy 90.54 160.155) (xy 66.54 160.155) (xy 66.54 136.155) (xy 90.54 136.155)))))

